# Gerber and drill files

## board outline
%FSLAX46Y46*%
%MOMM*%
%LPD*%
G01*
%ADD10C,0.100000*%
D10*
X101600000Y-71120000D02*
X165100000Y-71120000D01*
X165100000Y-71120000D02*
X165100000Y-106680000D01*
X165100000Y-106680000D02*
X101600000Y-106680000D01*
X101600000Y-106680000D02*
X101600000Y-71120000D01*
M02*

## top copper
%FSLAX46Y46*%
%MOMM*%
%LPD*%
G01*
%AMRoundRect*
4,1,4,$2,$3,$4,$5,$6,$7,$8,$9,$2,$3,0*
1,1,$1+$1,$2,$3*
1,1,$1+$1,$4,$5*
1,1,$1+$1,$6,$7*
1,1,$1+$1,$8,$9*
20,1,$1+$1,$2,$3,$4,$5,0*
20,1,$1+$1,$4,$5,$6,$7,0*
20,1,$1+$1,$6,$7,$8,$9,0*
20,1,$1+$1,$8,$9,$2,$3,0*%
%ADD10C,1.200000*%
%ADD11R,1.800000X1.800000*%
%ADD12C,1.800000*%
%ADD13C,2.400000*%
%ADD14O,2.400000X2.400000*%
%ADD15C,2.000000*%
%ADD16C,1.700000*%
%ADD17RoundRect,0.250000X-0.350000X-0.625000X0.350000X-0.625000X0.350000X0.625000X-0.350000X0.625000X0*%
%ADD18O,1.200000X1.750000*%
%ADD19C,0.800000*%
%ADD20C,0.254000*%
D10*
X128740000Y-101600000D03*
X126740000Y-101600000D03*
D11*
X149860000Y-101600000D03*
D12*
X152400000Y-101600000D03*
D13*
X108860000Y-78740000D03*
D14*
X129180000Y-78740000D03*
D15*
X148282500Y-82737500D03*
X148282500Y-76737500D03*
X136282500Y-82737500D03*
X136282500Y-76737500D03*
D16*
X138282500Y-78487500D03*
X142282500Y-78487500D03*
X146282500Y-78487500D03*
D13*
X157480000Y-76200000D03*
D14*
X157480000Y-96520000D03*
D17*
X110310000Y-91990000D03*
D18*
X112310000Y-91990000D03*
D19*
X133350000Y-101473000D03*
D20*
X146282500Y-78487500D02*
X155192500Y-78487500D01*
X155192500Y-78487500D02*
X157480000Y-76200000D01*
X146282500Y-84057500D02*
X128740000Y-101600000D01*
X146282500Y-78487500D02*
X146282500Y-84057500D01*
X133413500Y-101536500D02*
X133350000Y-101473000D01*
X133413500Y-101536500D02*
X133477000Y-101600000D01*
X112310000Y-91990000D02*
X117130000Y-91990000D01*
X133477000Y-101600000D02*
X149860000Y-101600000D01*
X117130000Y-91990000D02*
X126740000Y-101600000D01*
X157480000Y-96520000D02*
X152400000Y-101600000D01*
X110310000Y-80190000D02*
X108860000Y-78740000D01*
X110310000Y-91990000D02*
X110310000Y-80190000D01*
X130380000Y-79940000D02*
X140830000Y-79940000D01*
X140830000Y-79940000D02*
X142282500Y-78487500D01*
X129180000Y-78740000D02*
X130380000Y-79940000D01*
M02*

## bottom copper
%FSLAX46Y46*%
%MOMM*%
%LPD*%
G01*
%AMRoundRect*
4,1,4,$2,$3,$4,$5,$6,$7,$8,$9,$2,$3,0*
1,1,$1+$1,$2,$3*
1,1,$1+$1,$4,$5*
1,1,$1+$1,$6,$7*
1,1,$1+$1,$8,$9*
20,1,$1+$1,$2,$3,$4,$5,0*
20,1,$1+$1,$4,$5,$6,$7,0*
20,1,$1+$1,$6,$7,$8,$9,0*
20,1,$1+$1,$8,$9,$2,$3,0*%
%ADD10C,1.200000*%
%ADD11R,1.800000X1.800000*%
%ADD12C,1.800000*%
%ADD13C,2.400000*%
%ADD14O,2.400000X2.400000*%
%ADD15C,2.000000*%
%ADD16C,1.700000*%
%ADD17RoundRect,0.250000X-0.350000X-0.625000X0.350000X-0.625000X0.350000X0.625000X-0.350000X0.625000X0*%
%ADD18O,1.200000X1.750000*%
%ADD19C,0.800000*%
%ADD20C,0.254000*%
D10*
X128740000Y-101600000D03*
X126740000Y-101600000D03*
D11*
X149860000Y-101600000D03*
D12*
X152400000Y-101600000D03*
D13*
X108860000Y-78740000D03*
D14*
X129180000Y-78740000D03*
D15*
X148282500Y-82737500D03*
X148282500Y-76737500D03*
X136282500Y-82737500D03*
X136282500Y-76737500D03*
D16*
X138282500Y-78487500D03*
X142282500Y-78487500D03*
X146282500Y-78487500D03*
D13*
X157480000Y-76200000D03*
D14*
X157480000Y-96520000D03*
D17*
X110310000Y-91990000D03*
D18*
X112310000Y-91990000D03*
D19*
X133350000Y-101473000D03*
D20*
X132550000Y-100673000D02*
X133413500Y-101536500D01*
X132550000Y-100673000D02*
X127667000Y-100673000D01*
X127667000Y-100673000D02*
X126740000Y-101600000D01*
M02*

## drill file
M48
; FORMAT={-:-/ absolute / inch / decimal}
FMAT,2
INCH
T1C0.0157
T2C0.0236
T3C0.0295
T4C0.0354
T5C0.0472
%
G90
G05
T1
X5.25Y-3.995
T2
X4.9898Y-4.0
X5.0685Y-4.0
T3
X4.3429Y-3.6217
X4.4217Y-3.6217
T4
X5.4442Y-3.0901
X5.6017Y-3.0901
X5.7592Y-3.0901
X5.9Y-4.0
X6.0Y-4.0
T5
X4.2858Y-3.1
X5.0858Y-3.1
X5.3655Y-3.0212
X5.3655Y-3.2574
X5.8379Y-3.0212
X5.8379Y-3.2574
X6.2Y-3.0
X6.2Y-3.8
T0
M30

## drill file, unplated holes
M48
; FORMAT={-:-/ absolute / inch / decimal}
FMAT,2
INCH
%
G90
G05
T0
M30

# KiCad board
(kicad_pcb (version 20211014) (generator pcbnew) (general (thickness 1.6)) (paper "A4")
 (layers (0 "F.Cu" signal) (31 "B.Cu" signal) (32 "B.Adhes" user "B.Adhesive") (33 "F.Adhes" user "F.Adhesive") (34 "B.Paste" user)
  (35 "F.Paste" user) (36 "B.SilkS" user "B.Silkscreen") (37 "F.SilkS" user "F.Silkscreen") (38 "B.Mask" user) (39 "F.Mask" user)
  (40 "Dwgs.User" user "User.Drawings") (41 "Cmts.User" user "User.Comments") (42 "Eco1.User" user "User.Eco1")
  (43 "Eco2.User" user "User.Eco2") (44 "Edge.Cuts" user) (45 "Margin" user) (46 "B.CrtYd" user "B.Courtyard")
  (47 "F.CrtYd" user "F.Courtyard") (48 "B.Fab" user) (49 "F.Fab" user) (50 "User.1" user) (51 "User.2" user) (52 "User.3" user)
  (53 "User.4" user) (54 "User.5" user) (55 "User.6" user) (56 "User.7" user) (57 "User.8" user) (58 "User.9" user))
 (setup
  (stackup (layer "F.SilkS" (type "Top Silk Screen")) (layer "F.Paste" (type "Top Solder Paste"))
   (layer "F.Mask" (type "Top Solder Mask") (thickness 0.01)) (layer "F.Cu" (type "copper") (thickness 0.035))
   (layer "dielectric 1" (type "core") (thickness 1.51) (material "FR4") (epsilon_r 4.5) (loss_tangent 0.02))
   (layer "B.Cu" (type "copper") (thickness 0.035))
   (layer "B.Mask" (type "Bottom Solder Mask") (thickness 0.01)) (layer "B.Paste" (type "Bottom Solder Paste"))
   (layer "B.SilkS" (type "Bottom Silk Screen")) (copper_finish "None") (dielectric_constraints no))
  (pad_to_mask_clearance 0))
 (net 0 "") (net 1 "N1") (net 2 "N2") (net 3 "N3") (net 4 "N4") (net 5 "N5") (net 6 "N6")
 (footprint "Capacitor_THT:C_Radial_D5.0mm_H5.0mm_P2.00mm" (layer "F.Cu") (at 128.74 101.6 180)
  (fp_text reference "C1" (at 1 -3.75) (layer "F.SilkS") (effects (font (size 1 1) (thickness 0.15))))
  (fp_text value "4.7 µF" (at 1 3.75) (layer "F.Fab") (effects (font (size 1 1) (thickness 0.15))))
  (pad "1" thru_hole circle (at 0 0 180) (size 1.2 1.2) (drill 0.6) (layers *.Cu *.Mask) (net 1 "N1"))
  (pad "2" thru_hole circle (at 2 0 180) (size 1.2 1.2) (drill 0.6) (layers *.Cu *.Mask) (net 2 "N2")))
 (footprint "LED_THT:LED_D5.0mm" (layer "F.Cu") (at 149.86 101.6)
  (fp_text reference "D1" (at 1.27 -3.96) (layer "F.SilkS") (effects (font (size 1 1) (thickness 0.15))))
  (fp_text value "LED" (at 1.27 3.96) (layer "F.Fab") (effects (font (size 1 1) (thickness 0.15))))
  (pad "1" thru_hole rect (at 0 0) (size 1.8 1.8) (drill 0.9) (layers *.Cu *.Mask) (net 2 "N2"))
  (pad "2" thru_hole circle (at 2.54 0) (size 1.8 1.8) (drill 0.9) (layers *.Cu *.Mask) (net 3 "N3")))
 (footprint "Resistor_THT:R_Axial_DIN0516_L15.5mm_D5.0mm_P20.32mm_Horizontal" (layer "F.Cu") (at 108.86 78.74)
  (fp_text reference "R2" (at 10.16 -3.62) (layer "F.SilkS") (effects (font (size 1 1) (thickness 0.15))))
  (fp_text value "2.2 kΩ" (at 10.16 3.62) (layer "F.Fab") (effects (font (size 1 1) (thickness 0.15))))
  (pad "1" thru_hole circle (at 0 0) (size 2.4 2.4) (drill 1.2) (layers *.Cu *.Mask) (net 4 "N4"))
  (pad "2" thru_hole oval (at 20.32 0) (size 2.4 2.4) (drill 1.2) (layers *.Cu *.Mask) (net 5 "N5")))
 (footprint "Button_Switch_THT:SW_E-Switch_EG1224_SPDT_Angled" (layer "F.Cu") (at 138.2825 78.4875)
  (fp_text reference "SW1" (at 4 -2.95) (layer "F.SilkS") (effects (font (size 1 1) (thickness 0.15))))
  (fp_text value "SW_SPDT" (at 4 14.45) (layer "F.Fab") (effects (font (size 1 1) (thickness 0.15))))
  (pad "" thru_hole circle (at 10 4.25) (size 2 2) (drill 1.2) (layers *.Cu *.Mask))
  (pad "" thru_hole circle (at 10 -1.75) (size 2 2) (drill 1.2) (layers *.Cu *.Mask))
  (pad "" thru_hole circle (at -2 4.25) (size 2 2) (drill 1.2) (layers *.Cu *.Mask))
  (pad "" thru_hole circle (at -2 -1.75) (size 2 2) (drill 1.2) (layers *.Cu *.Mask))
  (pad "1" thru_hole circle (at 0 0) (size 1.7 1.7) (drill 0.9) (layers *.Cu *.Mask) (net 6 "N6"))
  (pad "2" thru_hole circle (at 4 0) (size 1.7 1.7) (drill 0.9) (layers *.Cu *.Mask) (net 5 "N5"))
  (pad "3" thru_hole circle (at 8 0) (size 1.7 1.7) (drill 0.9) (layers *.Cu *.Mask) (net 1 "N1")))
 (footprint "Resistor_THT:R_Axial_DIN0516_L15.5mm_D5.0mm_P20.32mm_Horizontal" (layer "F.Cu") (at 157.48 76.2 -90)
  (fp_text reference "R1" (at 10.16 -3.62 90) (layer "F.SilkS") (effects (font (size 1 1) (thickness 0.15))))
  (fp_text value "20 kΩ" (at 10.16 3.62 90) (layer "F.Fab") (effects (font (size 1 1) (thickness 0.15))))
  (pad "1" thru_hole circle (at 0 0 270) (size 2.4 2.4) (drill 1.2) (layers *.Cu *.Mask) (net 1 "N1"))
  (pad "2" thru_hole oval (at 20.32 0 270) (size 2.4 2.4) (drill 1.2) (layers *.Cu *.Mask) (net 3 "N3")))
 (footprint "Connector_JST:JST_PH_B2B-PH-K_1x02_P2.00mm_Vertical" (layer "F.Cu") (at 110.31 91.99)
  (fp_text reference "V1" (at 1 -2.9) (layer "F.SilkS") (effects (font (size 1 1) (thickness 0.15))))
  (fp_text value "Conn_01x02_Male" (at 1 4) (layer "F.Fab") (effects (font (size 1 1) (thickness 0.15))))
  (pad "1" thru_hole roundrect (at 0 0) (size 1.2 1.75) (drill 0.75) (layers *.Cu *.Mask) (roundrect_rratio 0.2083333333) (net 4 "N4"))
  (pad "2" thru_hole oval (at 2 0) (size 1.2 1.75) (drill 0.75) (layers *.Cu *.Mask) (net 2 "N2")))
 (gr_rect (start 101.6 71.12) (end 165.1 106.68) (layer "Edge.Cuts") (width 0.1) (fill none))
 (segment (start 146.2825 78.4875) (end 155.1925 78.4875) (width 0.254) (layer "F.Cu") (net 1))
 (segment (start 155.1925 78.4875) (end 157.48 76.2) (width 0.254) (layer "F.Cu") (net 1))
 (segment (start 146.2825 84.0575) (end 128.74 101.6) (width 0.254) (layer "F.Cu") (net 1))
 (segment (start 146.2825 78.4875) (end 146.2825 84.0575) (width 0.254) (layer "F.Cu") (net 1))
 (segment (start 133.4135 101.5365) (end 133.35 101.473) (width 0.254) (layer "F.Cu") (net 2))
 (segment (start 133.4135 101.5365) (end 133.477 101.6) (width 0.254) (layer "F.Cu") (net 2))
 (segment (start 112.31 91.99) (end 117.13 91.99) (width 0.254) (layer "F.Cu") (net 2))
 (segment (start 133.477 101.6) (end 149.86 101.6) (width 0.254) (layer "F.Cu") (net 2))
 (segment (start 117.13 91.99) (end 126.74 101.6) (width 0.254) (layer "F.Cu") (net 2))
 (via (at 133.35 101.473) (size 0.8) (drill 0.4) (layers "F.Cu" "B.Cu") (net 2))
 (segment (start 132.55 100.673) (end 133.4135 101.5365) (width 0.254) (layer "B.Cu") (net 2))
 (segment (start 132.55 100.673) (end 127.667 100.673) (width 0.254) (layer "B.Cu") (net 2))
 (segment (start 127.667 100.673) (end 126.74 101.6) (width 0.254) (layer "B.Cu") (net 2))
 (segment (start 157.48 96.52) (end 152.4 101.6) (width 0.254) (layer "F.Cu") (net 3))
 (segment (start 110.31 80.19) (end 108.86 78.74) (width 0.254) (layer "F.Cu") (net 4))
 (segment (start 110.31 91.99) (end 110.31 80.19) (width 0.254) (layer "F.Cu") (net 4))
 (segment (start 130.38 79.94) (end 140.83 79.94) (width 0.254) (layer "F.Cu") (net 5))
 (segment (start 140.83 79.94) (end 142.2825 78.4875) (width 0.254) (layer "F.Cu") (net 5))
 (segment (start 129.18 78.74) (end 130.38 79.94) (width 0.254) (layer "F.Cu") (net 5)))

